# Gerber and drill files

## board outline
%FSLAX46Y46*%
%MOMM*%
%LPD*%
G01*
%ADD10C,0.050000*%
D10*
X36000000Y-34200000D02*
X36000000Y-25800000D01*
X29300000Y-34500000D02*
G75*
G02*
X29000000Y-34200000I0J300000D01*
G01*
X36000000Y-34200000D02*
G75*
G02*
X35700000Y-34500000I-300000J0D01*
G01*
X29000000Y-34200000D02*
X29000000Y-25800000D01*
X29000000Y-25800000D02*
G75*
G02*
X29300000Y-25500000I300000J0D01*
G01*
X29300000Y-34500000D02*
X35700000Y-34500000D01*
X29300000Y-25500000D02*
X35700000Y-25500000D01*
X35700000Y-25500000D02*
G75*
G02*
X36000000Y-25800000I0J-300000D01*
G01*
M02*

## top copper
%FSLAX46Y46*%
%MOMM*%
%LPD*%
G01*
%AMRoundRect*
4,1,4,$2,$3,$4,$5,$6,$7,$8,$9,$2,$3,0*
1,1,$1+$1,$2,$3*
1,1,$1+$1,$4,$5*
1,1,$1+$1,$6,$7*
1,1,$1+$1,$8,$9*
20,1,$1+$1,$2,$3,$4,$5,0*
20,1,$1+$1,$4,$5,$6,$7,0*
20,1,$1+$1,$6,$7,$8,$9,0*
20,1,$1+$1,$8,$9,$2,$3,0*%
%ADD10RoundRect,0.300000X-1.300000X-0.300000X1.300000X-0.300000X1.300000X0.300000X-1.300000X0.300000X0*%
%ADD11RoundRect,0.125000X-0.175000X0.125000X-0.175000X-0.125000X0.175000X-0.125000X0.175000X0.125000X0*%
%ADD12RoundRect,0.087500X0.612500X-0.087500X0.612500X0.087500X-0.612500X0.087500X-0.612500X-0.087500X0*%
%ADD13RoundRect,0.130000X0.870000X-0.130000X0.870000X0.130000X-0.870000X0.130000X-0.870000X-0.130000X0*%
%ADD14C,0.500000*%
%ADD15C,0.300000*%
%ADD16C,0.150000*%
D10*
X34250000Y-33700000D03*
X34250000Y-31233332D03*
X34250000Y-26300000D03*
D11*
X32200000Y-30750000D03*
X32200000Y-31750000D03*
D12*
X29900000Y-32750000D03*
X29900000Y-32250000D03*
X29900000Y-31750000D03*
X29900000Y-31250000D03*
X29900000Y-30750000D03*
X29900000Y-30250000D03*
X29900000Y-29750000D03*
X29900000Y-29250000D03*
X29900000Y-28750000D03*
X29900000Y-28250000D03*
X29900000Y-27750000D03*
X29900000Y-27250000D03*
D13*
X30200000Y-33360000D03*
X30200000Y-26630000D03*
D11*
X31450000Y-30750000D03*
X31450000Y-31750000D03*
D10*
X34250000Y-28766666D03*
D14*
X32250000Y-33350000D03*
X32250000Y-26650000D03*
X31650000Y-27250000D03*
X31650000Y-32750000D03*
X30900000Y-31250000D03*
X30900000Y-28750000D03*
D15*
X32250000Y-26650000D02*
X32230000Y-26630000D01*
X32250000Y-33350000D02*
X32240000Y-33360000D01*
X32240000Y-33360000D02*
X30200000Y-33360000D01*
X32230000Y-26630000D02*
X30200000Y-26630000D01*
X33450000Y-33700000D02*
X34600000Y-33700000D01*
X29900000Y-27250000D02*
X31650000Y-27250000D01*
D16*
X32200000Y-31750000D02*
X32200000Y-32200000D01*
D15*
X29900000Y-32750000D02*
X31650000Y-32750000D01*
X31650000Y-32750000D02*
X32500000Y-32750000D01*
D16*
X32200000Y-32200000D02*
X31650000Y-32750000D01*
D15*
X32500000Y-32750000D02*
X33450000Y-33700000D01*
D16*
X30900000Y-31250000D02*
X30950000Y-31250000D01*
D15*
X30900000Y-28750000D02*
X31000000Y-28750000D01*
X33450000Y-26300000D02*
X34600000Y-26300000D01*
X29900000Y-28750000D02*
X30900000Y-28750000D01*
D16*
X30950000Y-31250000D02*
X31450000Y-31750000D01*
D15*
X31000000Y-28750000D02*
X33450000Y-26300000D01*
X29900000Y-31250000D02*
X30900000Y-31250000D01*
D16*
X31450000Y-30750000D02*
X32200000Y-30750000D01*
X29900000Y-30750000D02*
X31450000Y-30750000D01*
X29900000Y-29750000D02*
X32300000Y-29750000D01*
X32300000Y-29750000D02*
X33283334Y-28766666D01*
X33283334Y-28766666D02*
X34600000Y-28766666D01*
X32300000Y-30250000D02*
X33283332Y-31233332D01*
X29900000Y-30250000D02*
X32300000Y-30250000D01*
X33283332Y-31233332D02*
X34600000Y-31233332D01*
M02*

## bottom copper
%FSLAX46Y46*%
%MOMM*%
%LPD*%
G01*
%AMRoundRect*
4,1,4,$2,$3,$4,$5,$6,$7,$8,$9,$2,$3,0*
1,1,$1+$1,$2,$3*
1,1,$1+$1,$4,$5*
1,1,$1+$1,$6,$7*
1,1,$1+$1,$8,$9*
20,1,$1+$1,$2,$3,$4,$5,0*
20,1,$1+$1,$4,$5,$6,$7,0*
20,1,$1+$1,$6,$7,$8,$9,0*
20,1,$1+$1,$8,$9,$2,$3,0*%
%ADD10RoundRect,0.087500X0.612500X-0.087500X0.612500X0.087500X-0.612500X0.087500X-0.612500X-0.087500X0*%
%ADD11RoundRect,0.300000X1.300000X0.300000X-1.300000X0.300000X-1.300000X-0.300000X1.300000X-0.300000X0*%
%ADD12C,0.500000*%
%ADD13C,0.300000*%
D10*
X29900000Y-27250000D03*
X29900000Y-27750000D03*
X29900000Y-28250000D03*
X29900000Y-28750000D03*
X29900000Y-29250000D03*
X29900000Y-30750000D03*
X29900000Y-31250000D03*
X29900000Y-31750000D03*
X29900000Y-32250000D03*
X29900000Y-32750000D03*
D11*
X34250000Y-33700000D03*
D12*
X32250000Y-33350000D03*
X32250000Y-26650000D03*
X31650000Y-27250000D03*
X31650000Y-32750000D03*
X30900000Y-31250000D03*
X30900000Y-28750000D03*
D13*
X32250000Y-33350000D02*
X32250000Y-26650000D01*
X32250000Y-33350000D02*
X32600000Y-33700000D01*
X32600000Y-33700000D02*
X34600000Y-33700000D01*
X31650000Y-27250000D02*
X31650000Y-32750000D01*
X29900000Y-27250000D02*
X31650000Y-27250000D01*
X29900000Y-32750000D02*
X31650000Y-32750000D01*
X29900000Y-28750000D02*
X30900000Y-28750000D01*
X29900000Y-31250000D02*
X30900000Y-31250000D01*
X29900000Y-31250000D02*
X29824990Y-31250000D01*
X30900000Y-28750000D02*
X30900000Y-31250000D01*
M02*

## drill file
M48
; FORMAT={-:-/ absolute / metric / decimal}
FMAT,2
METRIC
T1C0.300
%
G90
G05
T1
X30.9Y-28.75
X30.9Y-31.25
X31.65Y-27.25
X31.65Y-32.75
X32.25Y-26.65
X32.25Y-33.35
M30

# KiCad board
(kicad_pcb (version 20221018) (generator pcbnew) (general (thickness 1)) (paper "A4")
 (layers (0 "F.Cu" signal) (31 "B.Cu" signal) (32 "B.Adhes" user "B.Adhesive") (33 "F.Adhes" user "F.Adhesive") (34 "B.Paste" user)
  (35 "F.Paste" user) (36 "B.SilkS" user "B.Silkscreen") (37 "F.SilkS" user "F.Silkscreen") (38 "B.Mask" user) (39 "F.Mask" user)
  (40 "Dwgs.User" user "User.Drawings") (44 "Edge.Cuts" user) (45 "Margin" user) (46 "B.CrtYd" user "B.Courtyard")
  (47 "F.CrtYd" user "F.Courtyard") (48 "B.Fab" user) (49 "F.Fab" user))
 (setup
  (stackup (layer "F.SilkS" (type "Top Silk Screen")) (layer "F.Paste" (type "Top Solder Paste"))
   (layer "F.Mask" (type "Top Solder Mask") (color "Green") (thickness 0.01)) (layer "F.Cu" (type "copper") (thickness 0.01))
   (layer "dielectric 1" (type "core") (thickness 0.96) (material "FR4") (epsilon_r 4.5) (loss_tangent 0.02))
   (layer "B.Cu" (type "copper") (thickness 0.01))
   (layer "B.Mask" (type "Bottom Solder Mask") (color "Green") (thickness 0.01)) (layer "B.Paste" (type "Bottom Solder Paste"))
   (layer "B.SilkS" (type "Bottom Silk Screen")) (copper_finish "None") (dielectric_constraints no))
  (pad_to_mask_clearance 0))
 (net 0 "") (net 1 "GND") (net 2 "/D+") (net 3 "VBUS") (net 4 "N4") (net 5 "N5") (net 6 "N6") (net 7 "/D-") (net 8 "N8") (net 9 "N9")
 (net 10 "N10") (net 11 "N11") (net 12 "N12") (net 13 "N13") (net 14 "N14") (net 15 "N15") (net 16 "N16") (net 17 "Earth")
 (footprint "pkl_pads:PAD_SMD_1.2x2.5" (layer "F.Cu") (at 34.6 33.7)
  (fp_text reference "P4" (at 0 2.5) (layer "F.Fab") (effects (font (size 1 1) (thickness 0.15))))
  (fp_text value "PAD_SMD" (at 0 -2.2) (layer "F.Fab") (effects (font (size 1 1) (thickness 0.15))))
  (pad "1" smd roundrect (at -0.35 0) (size 3.2 1.2) (layers "F.Cu" "F.Mask") (roundrect_rratio 0.25) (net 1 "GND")))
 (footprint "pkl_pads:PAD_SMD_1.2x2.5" (layer "F.Cu") (at 34.6 31.233332)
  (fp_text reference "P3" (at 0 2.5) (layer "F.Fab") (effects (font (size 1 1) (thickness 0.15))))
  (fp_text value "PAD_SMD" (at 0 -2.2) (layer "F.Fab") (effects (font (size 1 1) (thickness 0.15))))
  (pad "1" smd roundrect (at -0.35 0) (size 3.2 1.2) (layers "F.Cu" "F.Mask") (roundrect_rratio 0.25) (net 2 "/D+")))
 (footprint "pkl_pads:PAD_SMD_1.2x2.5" (layer "F.Cu") (at 34.6 26.3)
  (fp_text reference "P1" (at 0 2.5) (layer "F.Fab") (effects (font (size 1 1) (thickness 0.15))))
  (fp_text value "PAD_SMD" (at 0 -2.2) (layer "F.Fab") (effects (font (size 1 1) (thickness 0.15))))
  (pad "1" smd roundrect (at -0.35 0) (size 3.2 1.2) (layers "F.Cu" "F.Mask") (roundrect_rratio 0.25) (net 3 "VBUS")))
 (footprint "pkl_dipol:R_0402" (layer "F.Cu") (at 32.2 31.25 -90)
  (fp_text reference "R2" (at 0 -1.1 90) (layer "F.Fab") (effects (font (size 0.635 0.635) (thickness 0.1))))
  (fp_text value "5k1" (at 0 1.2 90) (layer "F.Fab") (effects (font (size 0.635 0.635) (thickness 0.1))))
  (pad "1" smd roundrect (at -0.5 0 270) (size 0.5 0.6) (layers "F.Cu" "F.Paste" "F.Mask") (roundrect_rratio 0.25) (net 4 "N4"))
  (pad "2" smd roundrect (at 0.5 0 270) (size 0.5 0.6) (layers "F.Cu" "F.Paste" "F.Mask") (roundrect_rratio 0.25) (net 1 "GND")))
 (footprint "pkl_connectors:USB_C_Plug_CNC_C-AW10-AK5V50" (layer "F.Cu") (at 30 30 90)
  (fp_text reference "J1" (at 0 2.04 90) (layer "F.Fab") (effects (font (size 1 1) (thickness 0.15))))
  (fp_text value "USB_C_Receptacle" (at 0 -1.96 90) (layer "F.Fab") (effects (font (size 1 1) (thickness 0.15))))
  (pad "A1" smd roundrect (at -2.75 -0.1 90) (size 0.35 1.4) (layers "F.Cu" "F.Paste" "F.Mask") (roundrect_rratio 0.25) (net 1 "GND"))
  (pad "A2" smd roundrect (at -2.25 -0.1 90) (size 0.35 1.4) (layers "F.Cu" "F.Paste" "F.Mask") (roundrect_rratio 0.25) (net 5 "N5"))
  (pad "A3" smd roundrect (at -1.75 -0.1 90) (size 0.35 1.4) (layers "F.Cu" "F.Paste" "F.Mask") (roundrect_rratio 0.25) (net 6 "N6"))
  (pad "A4" smd roundrect (at -1.25 -0.1 90) (size 0.35 1.4) (layers "F.Cu" "F.Paste" "F.Mask") (roundrect_rratio 0.25) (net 3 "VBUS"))
  (pad "A5" smd roundrect (at -0.75 -0.1 90) (size 0.35 1.4) (layers "F.Cu" "F.Paste" "F.Mask") (roundrect_rratio 0.25) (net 4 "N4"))
  (pad "A6" smd roundrect (at -0.25 -0.1 90) (size 0.35 1.4) (layers "F.Cu" "F.Paste" "F.Mask") (roundrect_rratio 0.25) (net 2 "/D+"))
  (pad "A7" smd roundrect (at 0.25 -0.1 90) (size 0.35 1.4) (layers "F.Cu" "F.Paste" "F.Mask") (roundrect_rratio 0.25) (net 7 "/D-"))
  (pad "A8" smd roundrect (at 0.75 -0.1 90) (size 0.35 1.4) (layers "F.Cu" "F.Paste" "F.Mask") (roundrect_rratio 0.25) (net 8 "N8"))
  (pad "A9" smd roundrect (at 1.25 -0.1 90) (size 0.35 1.4) (layers "F.Cu" "F.Paste" "F.Mask") (roundrect_rratio 0.25) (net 3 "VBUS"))
  (pad "A10" smd roundrect (at 1.75 -0.1 90) (size 0.35 1.4) (layers "F.Cu" "F.Paste" "F.Mask") (roundrect_rratio 0.25) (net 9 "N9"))
  (pad "A11" smd roundrect (at 2.25 -0.1 90) (size 0.35 1.4) (layers "F.Cu" "F.Paste" "F.Mask") (roundrect_rratio 0.25) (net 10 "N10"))
  (pad "A12" smd roundrect (at 2.75 -0.1 90) (size 0.35 1.4) (layers "F.Cu" "F.Paste" "F.Mask") (roundrect_rratio 0.25) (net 1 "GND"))
  (pad "B1" smd roundrect (at 2.75 -0.1 90) (size 0.35 1.4) (layers "B.Cu" "B.Paste" "B.Mask") (roundrect_rratio 0.25) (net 1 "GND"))
  (pad "B2" smd roundrect (at 2.25 -0.1 90) (size 0.35 1.4) (layers "B.Cu" "B.Paste" "B.Mask") (roundrect_rratio 0.25) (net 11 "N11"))
  (pad "B3" smd roundrect (at 1.75 -0.1 90) (size 0.35 1.4) (layers "B.Cu" "B.Paste" "B.Mask") (roundrect_rratio 0.25) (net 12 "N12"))
  (pad "B4" smd roundrect (at 1.25 -0.1 90) (size 0.35 1.4) (layers "B.Cu" "B.Paste" "B.Mask") (roundrect_rratio 0.25) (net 3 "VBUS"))
  (pad "B5" smd roundrect (at 0.75 -0.1 90) (size 0.35 1.4) (layers "B.Cu" "B.Paste" "B.Mask") (roundrect_rratio 0.25) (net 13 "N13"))
  (pad "B8" smd roundrect (at -0.75 -0.1 90) (size 0.35 1.4) (layers "B.Cu" "B.Paste" "B.Mask") (roundrect_rratio 0.25) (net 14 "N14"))
  (pad "B9" smd roundrect (at -1.25 -0.1 90) (size 0.35 1.4) (layers "B.Cu" "B.Paste" "B.Mask") (roundrect_rratio 0.25) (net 3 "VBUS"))
  (pad "B10" smd roundrect (at -1.75 -0.1 90) (size 0.35 1.4) (layers "B.Cu" "B.Paste" "B.Mask") (roundrect_rratio 0.25) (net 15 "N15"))
  (pad "B11" smd roundrect (at -2.25 -0.1 90) (size 0.35 1.4) (layers "B.Cu" "B.Paste" "B.Mask") (roundrect_rratio 0.25) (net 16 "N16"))
  (pad "B12" smd roundrect (at -2.75 -0.1 90) (size 0.35 1.4) (layers "B.Cu" "B.Paste" "B.Mask") (roundrect_rratio 0.25) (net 1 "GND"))
  (pad "S1" smd roundrect (at -3.36 0.2 90) (size 0.52 2) (layers "F.Cu" "F.Paste" "F.Mask") (roundrect_rratio 0.25) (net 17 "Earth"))
  (pad "S1" smd roundrect (at 3.37 0.2 90) (size 0.52 2) (layers "F.Cu" "F.Paste" "F.Mask") (roundrect_rratio 0.25) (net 17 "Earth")))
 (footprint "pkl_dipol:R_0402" (layer "F.Cu") (at 31.45 31.25 -90)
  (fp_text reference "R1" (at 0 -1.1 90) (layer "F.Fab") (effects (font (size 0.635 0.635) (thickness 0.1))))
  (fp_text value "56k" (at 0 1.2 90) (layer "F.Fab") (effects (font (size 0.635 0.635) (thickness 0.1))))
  (pad "1" smd roundrect (at -0.5 0 270) (size 0.5 0.6) (layers "F.Cu" "F.Paste" "F.Mask") (roundrect_rratio 0.25) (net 4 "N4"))
  (pad "2" smd roundrect (at 0.5 0 270) (size 0.5 0.6) (layers "F.Cu" "F.Paste" "F.Mask") (roundrect_rratio 0.25) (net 3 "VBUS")))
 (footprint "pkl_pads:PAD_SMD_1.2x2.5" (layer "F.Cu") (at 34.6 28.766666)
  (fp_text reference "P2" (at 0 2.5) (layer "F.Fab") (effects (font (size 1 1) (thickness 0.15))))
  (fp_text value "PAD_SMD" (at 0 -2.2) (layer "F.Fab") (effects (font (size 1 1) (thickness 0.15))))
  (pad "1" smd roundrect (at -0.35 0) (size 3.2 1.2) (layers "F.Cu" "F.Mask") (roundrect_rratio 0.25) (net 7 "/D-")))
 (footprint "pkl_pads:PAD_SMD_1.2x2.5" (layer "B.Cu") (at 34.6 33.7 180)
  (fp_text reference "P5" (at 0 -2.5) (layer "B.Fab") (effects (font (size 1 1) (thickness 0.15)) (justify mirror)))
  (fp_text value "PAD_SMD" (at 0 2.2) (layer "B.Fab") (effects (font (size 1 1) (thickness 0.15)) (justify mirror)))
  (pad "1" smd roundrect (at 0.35 0 180) (size 3.2 1.2) (layers "B.Cu" "B.Mask") (roundrect_rratio 0.25) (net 17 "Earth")))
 (gr_line (start 36 34.2) (end 36 25.8) (stroke (width 0.05) (type solid)) (layer "Edge.Cuts"))
 (gr_arc (start 29.3 34.5) (mid 29.087868 34.412132) (end 29 34.2) (stroke (width 0.05) (type solid)) (layer "Edge.Cuts"))
 (gr_arc (start 36 34.2) (mid 35.912132 34.412132) (end 35.7 34.5) (stroke (width 0.05) (type solid)) (layer "Edge.Cuts"))
 (gr_line (start 29 34.2) (end 29 25.8) (stroke (width 0.05) (type solid)) (layer "Edge.Cuts"))
 (gr_arc (start 29 25.8) (mid 29.087868 25.587868) (end 29.3 25.5) (stroke (width 0.05) (type solid)) (layer "Edge.Cuts"))
 (gr_line (start 29.3 34.5) (end 35.7 34.5) (stroke (width 0.05) (type solid)) (layer "Edge.Cuts"))
 (gr_line (start 29.3 25.5) (end 35.7 25.5) (stroke (width 0.05) (type solid)) (layer "Edge.Cuts"))
 (gr_arc (start 35.7 25.5) (mid 35.912132 25.587868) (end 36 25.8) (stroke (width 0.05) (type solid)) (layer "Edge.Cuts"))
 (segment (start 32.25 26.65) (end 32.23 26.63) (width 0.3) (layer "F.Cu") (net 17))
 (segment (start 32.25 33.35) (end 32.24 33.36) (width 0.3) (layer "F.Cu") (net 17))
 (segment (start 32.24 33.36) (end 30.2 33.36) (width 0.3) (layer "F.Cu") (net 17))
 (segment (start 32.23 26.63) (end 30.2 26.63) (width 0.3) (layer "F.Cu") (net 17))
 (via (at 32.25 33.35) (size 0.5) (drill 0.3) (layers "F.Cu" "B.Cu") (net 17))
 (via (at 32.25 26.65) (size 0.5) (drill 0.3) (layers "F.Cu" "B.Cu") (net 17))
 (segment (start 32.25 33.35) (end 32.25 26.65) (width 0.3) (layer "B.Cu") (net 17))
 (segment (start 32.25 33.35) (end 32.6 33.7) (width 0.3) (layer "B.Cu") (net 17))
 (segment (start 32.6 33.7) (end 34.6 33.7) (width 0.3) (layer "B.Cu") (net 17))
 (segment (start 33.45 33.7) (end 34.6 33.7) (width 0.3) (layer "F.Cu") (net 1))
 (segment (start 29.9 27.25) (end 31.65 27.25) (width 0.3) (layer "F.Cu") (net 1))
 (segment (start 32.2 31.75) (end 32.2 32.2) (width 0.15) (layer "F.Cu") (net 1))
 (segment (start 29.9 32.75) (end 31.65 32.75) (width 0.3) (layer "F.Cu") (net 1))
 (segment (start 31.65 32.75) (end 32.5 32.75) (width 0.3) (layer "F.Cu") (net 1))
 (segment (start 32.2 32.2) (end 31.65 32.75) (width 0.15) (layer "F.Cu") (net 1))
 (segment (start 32.5 32.75) (end 33.45 33.7) (width 0.3) (layer "F.Cu") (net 1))
 (via (at 31.65 27.25) (size 0.5) (drill 0.3) (layers "F.Cu" "B.Cu") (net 1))
 (via (at 31.65 32.75) (size 0.5) (drill 0.3) (layers "F.Cu" "B.Cu") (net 1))
 (segment (start 31.65 27.25) (end 31.65 32.75) (width 0.3) (layer "B.Cu") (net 1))
 (segment (start 29.9 27.25) (end 31.65 27.25) (width 0.3) (layer "B.Cu") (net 1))
 (segment (start 29.9 32.75) (end 31.65 32.75) (width 0.3) (layer "B.Cu") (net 1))
 (segment (start 30.9 31.25) (end 30.95 31.25) (width 0.15) (layer "F.Cu") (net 3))
 (segment (start 30.9 28.75) (end 31 28.75) (width 0.3) (layer "F.Cu") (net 3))
 (segment (start 33.45 26.3) (end 34.6 26.3) (width 0.3) (layer "F.Cu") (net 3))
 (segment (start 29.9 28.75) (end 30.9 28.75) (width 0.3) (layer "F.Cu") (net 3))
 (segment (start 30.95 31.25) (end 31.45 31.75) (width 0.15) (layer "F.Cu") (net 3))
 (segment (start 31 28.75) (end 33.45 26.3) (width 0.3) (layer "F.Cu") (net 3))
 (segment (start 29.9 31.25) (end 30.9 31.25) (width 0.3) (layer "F.Cu") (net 3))
 (via (at 30.9 31.25) (size 0.5) (drill 0.3) (layers "F.Cu" "B.Cu") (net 3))
 (via (at 30.9 28.75) (size 0.5) (drill 0.3) (layers "F.Cu" "B.Cu") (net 3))
 (segment (start 29.9 28.75) (end 30.9 28.75) (width 0.3) (layer "B.Cu") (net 3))
 (segment (start 29.9 31.25) (end 30.9 31.25) (width 0.3) (layer "B.Cu") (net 3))
 (segment (start 29.9 31.25) (end 29.82499 31.25) (width 0.3) (layer "B.Cu") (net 3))
 (segment (start 30.9 28.75) (end 30.9 31.25) (width 0.3) (layer "B.Cu") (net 3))
 (segment (start 31.45 30.75) (end 32.2 30.75) (width 0.15) (layer "F.Cu") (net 4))
 (segment (start 29.9 30.75) (end 31.45 30.75) (width 0.15) (layer "F.Cu") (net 4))
 (segment (start 29.9 29.75) (end 32.3 29.75) (width 0.15) (layer "F.Cu") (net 7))
 (segment (start 32.3 29.75) (end 33.283334 28.766666) (width 0.15) (layer "F.Cu") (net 7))
 (segment (start 33.283334 28.766666) (end 34.6 28.766666) (width 0.15) (layer "F.Cu") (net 7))
 (segment (start 32.3 30.25) (end 33.283332 31.233332) (width 0.15) (layer "F.Cu") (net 2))
 (segment (start 29.9 30.25) (end 32.3 30.25) (width 0.15) (layer "F.Cu") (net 2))
 (segment (start 33.283332 31.233332) (end 34.6 31.233332) (width 0.15) (layer "F.Cu") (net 2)))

